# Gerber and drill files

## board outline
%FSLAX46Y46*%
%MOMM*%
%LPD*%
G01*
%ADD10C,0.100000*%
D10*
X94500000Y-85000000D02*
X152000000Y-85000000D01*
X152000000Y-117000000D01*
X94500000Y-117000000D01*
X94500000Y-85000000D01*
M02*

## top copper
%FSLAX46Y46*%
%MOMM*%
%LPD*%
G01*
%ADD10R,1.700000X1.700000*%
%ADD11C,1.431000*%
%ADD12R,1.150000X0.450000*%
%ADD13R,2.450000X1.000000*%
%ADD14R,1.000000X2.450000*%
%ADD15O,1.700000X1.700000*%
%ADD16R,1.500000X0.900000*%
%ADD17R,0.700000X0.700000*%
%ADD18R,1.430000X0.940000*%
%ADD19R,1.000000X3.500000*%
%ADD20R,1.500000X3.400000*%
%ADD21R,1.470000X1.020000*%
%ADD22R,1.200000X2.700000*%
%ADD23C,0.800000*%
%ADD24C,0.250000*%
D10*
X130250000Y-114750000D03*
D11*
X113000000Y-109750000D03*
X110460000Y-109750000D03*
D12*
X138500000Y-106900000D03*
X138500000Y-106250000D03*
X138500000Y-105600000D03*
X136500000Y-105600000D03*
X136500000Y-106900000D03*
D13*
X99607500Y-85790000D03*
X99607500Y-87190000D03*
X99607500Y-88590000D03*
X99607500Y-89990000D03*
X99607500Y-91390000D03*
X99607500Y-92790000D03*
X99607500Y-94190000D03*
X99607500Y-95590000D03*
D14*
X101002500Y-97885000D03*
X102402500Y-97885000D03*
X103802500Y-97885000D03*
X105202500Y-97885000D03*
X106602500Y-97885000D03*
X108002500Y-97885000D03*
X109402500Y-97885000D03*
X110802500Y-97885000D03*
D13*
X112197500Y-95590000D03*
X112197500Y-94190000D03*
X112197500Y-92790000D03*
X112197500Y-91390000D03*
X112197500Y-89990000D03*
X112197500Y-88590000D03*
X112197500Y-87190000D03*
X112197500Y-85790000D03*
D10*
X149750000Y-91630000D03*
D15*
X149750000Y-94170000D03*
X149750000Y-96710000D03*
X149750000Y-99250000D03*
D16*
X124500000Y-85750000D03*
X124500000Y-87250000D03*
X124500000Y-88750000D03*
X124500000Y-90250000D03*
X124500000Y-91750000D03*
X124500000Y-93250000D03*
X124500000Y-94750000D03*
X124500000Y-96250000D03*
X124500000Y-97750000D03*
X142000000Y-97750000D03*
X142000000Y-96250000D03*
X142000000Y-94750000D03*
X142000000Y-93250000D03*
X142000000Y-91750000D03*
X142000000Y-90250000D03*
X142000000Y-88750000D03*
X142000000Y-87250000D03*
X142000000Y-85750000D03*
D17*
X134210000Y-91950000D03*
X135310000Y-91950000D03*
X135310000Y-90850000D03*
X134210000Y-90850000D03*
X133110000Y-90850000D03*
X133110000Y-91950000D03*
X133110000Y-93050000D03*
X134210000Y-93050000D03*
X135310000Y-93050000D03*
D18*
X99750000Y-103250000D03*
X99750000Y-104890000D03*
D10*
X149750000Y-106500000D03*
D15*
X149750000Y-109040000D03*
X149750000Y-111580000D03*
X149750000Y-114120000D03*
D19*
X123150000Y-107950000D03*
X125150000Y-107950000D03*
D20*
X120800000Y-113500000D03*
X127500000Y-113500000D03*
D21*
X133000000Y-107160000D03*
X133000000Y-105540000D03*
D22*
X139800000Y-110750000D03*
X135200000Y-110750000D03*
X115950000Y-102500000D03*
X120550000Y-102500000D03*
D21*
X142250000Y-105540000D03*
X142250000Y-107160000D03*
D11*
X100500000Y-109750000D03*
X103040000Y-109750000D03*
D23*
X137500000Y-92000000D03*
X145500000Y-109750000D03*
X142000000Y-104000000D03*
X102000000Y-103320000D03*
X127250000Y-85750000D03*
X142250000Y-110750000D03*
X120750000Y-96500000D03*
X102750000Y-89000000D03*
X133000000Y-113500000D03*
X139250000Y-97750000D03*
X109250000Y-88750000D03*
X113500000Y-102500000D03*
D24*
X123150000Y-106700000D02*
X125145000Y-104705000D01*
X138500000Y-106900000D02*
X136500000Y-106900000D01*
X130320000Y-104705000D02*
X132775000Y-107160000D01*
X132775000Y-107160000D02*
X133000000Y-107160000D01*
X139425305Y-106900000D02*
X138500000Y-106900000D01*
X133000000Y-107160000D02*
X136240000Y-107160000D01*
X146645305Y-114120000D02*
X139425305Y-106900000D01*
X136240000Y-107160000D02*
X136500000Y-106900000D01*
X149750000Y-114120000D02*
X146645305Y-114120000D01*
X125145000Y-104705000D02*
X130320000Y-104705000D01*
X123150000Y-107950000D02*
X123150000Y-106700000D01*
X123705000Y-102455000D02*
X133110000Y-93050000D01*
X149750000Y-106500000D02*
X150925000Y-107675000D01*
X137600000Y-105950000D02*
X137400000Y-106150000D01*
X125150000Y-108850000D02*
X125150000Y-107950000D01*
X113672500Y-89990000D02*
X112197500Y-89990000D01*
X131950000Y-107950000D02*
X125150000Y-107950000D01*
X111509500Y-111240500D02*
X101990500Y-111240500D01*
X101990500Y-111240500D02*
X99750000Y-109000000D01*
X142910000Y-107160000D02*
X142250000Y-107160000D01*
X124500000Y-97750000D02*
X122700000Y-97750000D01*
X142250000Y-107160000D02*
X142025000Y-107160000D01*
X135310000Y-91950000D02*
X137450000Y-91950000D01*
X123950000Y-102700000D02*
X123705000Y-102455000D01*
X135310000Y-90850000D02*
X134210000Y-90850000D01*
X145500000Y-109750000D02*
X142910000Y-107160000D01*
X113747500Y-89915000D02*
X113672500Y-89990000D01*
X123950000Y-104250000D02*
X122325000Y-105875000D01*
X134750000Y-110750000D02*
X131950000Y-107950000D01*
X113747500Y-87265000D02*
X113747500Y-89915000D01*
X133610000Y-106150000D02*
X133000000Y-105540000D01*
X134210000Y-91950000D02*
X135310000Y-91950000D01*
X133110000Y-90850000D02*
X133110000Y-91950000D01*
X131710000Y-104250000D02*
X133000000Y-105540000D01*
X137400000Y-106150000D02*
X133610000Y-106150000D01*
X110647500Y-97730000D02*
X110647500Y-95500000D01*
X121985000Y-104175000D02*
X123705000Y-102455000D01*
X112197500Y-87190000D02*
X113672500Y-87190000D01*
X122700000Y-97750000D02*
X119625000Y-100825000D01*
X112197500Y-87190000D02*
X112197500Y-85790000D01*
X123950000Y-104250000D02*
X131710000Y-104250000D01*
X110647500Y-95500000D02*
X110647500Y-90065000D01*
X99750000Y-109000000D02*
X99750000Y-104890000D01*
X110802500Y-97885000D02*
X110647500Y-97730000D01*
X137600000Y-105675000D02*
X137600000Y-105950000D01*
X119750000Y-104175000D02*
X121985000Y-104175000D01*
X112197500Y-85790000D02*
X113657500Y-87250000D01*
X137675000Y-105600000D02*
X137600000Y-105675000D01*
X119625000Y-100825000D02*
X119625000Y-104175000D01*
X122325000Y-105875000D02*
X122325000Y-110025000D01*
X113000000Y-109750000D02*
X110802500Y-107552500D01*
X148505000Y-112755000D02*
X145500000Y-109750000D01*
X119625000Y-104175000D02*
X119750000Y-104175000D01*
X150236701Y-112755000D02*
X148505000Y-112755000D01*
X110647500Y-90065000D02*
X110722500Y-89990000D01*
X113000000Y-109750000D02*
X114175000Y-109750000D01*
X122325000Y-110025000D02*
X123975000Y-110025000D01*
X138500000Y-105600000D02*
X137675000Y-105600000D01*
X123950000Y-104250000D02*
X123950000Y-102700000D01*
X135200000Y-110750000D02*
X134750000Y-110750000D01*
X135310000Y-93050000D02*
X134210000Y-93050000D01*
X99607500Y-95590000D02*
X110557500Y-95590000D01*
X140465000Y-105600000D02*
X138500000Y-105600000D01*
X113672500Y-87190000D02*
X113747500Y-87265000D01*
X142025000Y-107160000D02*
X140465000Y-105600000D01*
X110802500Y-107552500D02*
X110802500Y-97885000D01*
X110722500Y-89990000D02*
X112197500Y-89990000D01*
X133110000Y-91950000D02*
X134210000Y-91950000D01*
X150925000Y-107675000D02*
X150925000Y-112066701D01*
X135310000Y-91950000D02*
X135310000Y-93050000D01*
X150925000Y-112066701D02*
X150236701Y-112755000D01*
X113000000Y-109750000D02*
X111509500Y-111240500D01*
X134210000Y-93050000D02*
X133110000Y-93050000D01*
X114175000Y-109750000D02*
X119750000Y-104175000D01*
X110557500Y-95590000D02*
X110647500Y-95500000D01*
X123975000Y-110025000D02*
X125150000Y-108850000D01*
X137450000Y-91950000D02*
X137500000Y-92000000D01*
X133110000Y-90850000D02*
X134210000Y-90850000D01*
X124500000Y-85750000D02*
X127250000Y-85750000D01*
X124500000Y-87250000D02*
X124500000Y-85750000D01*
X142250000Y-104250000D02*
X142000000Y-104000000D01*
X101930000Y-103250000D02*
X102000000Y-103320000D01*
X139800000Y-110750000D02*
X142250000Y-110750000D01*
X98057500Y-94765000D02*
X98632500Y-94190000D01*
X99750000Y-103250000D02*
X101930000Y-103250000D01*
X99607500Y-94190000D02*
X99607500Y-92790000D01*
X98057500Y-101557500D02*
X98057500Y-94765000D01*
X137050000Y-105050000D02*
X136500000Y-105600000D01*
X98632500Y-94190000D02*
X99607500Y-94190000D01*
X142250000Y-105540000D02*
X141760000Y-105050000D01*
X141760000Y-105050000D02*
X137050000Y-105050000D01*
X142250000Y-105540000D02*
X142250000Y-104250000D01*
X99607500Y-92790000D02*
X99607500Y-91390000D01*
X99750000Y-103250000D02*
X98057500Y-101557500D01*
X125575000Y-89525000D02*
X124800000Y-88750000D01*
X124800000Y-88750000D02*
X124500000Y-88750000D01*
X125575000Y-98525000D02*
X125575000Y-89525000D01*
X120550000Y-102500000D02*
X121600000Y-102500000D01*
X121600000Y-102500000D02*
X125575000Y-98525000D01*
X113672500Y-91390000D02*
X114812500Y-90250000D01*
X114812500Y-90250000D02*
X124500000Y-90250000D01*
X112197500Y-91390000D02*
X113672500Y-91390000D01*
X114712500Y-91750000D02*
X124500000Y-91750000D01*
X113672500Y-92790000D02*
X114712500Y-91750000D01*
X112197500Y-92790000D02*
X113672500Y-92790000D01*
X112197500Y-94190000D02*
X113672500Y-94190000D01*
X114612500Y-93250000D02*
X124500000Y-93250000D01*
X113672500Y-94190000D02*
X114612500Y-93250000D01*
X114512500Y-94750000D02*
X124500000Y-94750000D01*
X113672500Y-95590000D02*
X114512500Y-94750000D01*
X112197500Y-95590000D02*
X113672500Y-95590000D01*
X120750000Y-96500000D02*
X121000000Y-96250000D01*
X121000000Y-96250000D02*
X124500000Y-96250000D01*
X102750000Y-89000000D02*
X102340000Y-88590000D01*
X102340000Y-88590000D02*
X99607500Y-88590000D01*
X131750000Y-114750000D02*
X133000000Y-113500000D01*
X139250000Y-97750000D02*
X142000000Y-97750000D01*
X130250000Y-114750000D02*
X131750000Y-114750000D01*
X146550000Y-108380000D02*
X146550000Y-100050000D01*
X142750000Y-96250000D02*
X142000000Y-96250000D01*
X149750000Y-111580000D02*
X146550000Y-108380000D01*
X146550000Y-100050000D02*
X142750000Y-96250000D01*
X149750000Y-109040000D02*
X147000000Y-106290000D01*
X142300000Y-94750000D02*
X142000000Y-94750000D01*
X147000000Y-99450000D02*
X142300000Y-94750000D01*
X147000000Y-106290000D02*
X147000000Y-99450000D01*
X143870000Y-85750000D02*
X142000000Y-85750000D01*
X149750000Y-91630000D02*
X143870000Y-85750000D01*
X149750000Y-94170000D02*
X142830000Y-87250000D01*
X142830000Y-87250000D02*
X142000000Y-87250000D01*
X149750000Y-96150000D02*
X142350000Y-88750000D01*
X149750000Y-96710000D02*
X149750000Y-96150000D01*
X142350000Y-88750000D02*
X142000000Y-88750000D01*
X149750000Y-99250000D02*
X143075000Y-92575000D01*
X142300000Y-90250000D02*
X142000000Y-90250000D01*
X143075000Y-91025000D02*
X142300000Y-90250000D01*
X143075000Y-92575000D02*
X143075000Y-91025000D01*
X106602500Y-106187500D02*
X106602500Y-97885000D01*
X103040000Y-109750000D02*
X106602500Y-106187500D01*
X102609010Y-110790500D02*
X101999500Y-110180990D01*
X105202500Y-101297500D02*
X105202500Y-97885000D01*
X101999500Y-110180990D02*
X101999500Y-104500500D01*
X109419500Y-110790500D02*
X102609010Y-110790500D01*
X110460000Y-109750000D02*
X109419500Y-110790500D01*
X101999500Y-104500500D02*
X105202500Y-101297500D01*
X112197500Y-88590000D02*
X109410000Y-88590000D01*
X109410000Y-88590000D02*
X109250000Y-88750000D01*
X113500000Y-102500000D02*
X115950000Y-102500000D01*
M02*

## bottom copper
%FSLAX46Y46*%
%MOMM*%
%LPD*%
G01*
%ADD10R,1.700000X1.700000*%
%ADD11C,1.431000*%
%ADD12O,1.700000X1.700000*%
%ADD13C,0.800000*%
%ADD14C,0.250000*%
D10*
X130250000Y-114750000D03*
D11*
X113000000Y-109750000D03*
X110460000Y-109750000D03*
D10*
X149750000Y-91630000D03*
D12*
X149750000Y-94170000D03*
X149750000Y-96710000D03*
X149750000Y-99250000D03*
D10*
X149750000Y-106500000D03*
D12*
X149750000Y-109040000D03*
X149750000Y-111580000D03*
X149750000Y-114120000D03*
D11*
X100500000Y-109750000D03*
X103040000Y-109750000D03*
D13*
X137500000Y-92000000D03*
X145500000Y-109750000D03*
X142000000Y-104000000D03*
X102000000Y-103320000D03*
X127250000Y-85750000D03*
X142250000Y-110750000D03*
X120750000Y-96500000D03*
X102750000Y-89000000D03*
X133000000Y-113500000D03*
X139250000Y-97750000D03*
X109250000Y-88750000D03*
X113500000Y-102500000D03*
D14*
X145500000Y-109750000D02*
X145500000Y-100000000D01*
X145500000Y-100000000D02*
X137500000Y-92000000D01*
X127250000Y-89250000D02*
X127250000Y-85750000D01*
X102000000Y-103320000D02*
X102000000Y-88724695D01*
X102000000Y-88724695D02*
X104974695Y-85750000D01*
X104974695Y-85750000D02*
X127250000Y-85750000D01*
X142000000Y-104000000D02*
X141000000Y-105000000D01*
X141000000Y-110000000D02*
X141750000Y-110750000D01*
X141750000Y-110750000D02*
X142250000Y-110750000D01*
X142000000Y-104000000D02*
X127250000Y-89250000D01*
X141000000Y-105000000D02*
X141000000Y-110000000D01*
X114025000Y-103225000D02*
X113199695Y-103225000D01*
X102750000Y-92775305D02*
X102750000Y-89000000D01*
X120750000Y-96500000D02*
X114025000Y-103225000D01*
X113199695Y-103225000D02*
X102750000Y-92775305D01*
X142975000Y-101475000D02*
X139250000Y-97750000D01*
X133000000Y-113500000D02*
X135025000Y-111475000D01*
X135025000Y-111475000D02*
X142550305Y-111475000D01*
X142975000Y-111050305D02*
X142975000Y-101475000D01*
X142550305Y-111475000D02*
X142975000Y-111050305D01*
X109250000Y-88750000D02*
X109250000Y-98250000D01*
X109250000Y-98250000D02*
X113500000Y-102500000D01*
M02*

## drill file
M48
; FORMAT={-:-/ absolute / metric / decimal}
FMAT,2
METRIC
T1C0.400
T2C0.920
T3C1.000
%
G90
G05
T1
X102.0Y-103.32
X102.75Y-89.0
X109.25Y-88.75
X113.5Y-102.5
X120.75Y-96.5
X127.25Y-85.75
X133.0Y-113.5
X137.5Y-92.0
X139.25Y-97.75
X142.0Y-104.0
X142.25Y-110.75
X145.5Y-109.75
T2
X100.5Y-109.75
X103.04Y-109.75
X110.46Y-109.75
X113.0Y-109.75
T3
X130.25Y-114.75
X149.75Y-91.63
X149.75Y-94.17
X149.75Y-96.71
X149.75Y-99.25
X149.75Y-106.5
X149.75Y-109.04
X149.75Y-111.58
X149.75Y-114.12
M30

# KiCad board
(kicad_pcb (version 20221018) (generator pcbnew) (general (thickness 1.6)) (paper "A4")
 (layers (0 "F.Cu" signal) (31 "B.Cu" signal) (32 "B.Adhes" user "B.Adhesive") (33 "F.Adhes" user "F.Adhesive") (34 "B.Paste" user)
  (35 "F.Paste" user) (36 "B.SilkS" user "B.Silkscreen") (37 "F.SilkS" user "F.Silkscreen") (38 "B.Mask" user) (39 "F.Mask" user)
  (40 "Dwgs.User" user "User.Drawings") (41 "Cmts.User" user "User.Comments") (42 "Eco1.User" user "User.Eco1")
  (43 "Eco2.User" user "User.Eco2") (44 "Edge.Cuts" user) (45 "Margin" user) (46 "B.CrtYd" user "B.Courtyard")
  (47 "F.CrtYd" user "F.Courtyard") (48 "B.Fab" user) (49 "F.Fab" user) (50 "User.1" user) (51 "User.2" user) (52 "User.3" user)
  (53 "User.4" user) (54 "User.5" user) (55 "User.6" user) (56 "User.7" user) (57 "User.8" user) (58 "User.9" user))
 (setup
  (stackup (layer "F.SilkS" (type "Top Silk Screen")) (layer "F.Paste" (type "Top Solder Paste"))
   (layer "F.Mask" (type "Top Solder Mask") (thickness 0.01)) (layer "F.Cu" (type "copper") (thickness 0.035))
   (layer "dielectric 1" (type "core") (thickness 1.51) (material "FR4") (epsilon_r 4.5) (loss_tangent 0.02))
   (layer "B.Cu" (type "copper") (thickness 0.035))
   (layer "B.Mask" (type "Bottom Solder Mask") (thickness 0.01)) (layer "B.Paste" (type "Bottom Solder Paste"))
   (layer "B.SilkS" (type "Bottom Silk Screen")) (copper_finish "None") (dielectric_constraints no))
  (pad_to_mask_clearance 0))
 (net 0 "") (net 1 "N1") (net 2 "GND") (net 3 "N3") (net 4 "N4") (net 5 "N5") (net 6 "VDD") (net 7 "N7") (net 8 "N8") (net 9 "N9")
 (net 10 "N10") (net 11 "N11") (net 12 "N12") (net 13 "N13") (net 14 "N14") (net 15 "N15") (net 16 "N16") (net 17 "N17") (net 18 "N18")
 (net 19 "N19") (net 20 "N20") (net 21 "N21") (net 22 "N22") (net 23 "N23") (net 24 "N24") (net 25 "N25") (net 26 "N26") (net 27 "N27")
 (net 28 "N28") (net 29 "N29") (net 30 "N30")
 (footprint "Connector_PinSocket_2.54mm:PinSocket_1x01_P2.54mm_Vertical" (layer "F.Cu") (at 130.25 114.75)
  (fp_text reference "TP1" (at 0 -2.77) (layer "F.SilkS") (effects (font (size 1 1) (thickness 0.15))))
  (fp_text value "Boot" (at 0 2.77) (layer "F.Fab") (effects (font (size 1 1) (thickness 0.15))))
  (pad "1" thru_hole rect (at 0 0) (size 1.7 1.7) (drill 1) (layers "*.Cu" "*.Mask") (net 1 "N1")))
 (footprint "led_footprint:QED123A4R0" (layer "F.Cu") (at 113 109.75)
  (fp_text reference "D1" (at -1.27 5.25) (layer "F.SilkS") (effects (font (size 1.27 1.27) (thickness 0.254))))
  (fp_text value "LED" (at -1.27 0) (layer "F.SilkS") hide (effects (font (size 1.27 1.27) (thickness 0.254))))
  (pad "1" thru_hole circle (at 0 0) (size 1.431 1.431) (drill 0.92) (layers "*.Cu" "*.Mask") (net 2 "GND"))
  (pad "2" thru_hole circle (at -2.54 0) (size 1.431 1.431) (drill 0.92) (layers "*.Cu" "*.Mask") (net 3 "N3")))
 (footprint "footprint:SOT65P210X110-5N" (layer "F.Cu") (at 137.5 106.25 180)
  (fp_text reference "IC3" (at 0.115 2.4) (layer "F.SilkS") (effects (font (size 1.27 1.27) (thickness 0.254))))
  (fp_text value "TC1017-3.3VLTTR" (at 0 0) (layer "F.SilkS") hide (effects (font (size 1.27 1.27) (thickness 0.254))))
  (pad "1" smd rect (at -1 -0.65 270) (size 0.45 1.15) (layers "F.Cu" "F.Paste" "F.Mask") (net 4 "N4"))
  (pad "2" smd rect (at -1 0 270) (size 0.45 1.15) (layers "F.Cu" "F.Paste" "F.Mask") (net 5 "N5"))
  (pad "3" smd rect (at -1 0.65 270) (size 0.45 1.15) (layers "F.Cu" "F.Paste" "F.Mask") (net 2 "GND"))
  (pad "4" smd rect (at 1 0.65 270) (size 0.45 1.15) (layers "F.Cu" "F.Paste" "F.Mask") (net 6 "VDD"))
  (pad "5" smd rect (at 1 -0.65 270) (size 0.45 1.15) (layers "F.Cu" "F.Paste" "F.Mask") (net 4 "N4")))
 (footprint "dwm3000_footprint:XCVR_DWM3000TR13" (layer "F.Cu") (at 105.9025 86.74)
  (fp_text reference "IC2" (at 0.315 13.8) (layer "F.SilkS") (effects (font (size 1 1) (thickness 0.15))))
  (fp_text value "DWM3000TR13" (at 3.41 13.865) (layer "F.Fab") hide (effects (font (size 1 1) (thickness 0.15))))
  (pad "1" smd rect (at -6.295 -0.95) (size 2.45 1) (layers "F.Cu" "F.Paste" "F.Mask") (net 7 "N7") (solder_mask_margin 0.102))
  (pad "2" smd rect (at -6.295 0.45) (size 2.45 1) (layers "F.Cu" "F.Paste" "F.Mask") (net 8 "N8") (solder_mask_margin 0.102))
  (pad "3" smd rect (at -6.295 1.85) (size 2.45 1) (layers "F.Cu" "F.Paste" "F.Mask") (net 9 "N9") (solder_mask_margin 0.102))
  (pad "4" smd rect (at -6.295 3.25) (size 2.45 1) (layers "F.Cu" "F.Paste" "F.Mask") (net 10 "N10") (solder_mask_margin 0.102))
  (pad "5" smd rect (at -6.295 4.65) (size 2.45 1) (layers "F.Cu" "F.Paste" "F.Mask") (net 6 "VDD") (solder_mask_margin 0.102))
  (pad "6" smd rect (at -6.295 6.05) (size 2.45 1) (layers "F.Cu" "F.Paste" "F.Mask") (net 6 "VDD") (solder_mask_margin 0.102))
  (pad "7" smd rect (at -6.295 7.45) (size 2.45 1) (layers "F.Cu" "F.Paste" "F.Mask") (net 6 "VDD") (solder_mask_margin 0.102))
  (pad "8" smd rect (at -6.295 8.85) (size 2.45 1) (layers "F.Cu" "F.Paste" "F.Mask") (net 2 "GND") (solder_mask_margin 0.102))
  (pad "9" smd rect (at -4.9 11.145) (size 1 2.45) (layers "F.Cu" "F.Paste" "F.Mask") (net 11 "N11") (solder_mask_margin 0.102))
  (pad "10" smd rect (at -3.5 11.145) (size 1 2.45) (layers "F.Cu" "F.Paste" "F.Mask") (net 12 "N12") (solder_mask_margin 0.102))
  (pad "11" smd rect (at -2.1 11.145) (size 1 2.45) (layers "F.Cu" "F.Paste" "F.Mask") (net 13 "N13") (solder_mask_margin 0.102))
  (pad "12" smd rect (at -0.7 11.145) (size 1 2.45) (layers "F.Cu" "F.Paste" "F.Mask") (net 3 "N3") (solder_mask_margin 0.102))
  (pad "13" smd rect (at 0.7 11.145) (size 1 2.45) (layers "F.Cu" "F.Paste" "F.Mask") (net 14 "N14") (solder_mask_margin 0.102))
  (pad "14" smd rect (at 2.1 11.145) (size 1 2.45) (layers "F.Cu" "F.Paste" "F.Mask") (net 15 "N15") (solder_mask_margin 0.102))
  (pad "15" smd rect (at 3.5 11.145) (size 1 2.45) (layers "F.Cu" "F.Paste" "F.Mask") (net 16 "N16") (solder_mask_margin 0.102))
  (pad "16" smd rect (at 4.9 11.145) (size 1 2.45) (layers "F.Cu" "F.Paste" "F.Mask") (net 2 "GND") (solder_mask_margin 0.102))
  (pad "17" smd rect (at 6.295 8.85) (size 2.45 1) (layers "F.Cu" "F.Paste" "F.Mask") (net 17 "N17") (solder_mask_margin 0.102))
  (pad "18" smd rect (at 6.295 7.45) (size 2.45 1) (layers "F.Cu" "F.Paste" "F.Mask") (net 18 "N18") (solder_mask_margin 0.102))
  (pad "19" smd rect (at 6.295 6.05) (size 2.45 1) (layers "F.Cu" "F.Paste" "F.Mask") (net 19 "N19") (solder_mask_margin 0.102))
  (pad "20" smd rect (at 6.295 4.65) (size 2.45 1) (layers "F.Cu" "F.Paste" "F.Mask") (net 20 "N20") (solder_mask_margin 0.102))
  (pad "21" smd rect (at 6.295 3.25) (size 2.45 1) (layers "F.Cu" "F.Paste" "F.Mask") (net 2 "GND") (solder_mask_margin 0.102))
  (pad "22" smd rect (at 6.295 1.85) (size 2.45 1) (layers "F.Cu" "F.Paste" "F.Mask") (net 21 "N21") (solder_mask_margin 0.102))
  (pad "23" smd rect (at 6.295 0.45) (size 2.45 1) (layers "F.Cu" "F.Paste" "F.Mask") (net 2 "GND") (solder_mask_margin 0.102))
  (pad "24" smd rect (at 6.295 -0.95) (size 2.45 1) (layers "F.Cu" "F.Paste" "F.Mask") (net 2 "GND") (solder_mask_margin 0.102))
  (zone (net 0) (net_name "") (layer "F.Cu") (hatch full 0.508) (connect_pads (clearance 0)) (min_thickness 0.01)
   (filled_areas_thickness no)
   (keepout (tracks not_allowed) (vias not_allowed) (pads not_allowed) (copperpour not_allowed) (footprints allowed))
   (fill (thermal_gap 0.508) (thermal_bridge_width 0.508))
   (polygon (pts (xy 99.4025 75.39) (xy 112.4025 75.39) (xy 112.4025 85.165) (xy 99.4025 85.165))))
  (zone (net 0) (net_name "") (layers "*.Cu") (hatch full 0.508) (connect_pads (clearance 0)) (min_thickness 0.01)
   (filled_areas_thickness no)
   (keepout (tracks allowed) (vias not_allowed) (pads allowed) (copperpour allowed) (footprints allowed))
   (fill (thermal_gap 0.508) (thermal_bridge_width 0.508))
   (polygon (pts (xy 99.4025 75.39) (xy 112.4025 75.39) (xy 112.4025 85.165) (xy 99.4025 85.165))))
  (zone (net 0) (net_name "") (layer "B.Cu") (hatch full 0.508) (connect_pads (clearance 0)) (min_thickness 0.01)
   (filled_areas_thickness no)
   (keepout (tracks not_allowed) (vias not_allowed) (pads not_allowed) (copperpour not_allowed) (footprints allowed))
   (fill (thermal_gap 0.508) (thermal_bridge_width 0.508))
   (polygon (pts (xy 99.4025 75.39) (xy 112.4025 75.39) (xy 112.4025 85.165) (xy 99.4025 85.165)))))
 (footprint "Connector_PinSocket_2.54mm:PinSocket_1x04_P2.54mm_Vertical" (layer "F.Cu") (at 149.75 91.63)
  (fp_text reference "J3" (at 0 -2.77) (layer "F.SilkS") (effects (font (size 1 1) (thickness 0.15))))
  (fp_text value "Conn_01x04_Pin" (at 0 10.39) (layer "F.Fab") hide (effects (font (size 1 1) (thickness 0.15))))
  (pad "1" thru_hole rect (at 0 0) (size 1.7 1.7) (drill 1) (layers "*.Cu" "*.Mask") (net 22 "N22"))
  (pad "2" thru_hole oval (at 0 2.54) (size 1.7 1.7) (drill 1) (layers "*.Cu" "*.Mask") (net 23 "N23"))
  (pad "3" thru_hole oval (at 0 5.08) (size 1.7 1.7) (drill 1) (layers "*.Cu" "*.Mask") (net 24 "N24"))
  (pad "4" thru_hole oval (at 0 7.62) (size 1.7 1.7) (drill 1) (layers "*.Cu" "*.Mask") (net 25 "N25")))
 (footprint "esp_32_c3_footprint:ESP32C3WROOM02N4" (layer "F.Cu") (at 134.21 91.95)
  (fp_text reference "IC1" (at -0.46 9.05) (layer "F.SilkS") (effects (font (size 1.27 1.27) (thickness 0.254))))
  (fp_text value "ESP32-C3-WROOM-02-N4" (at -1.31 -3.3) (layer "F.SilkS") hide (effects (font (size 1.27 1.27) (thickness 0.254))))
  (pad "1" smd rect (at -9.71 -6.2 90) (size 0.9 1.5) (layers "F.Cu" "F.Paste" "F.Mask") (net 6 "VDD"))
  (pad "2" smd rect (at -9.71 -4.7 90) (size 0.9 1.5) (layers "F.Cu" "F.Paste" "F.Mask") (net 6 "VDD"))
  (pad "3" smd rect (at -9.71 -3.2 90) (size 0.9 1.5) (layers "F.Cu" "F.Paste" "F.Mask") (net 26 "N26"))
  (pad "4" smd rect (at -9.71 -1.7 90) (size 0.9 1.5) (layers "F.Cu" "F.Paste" "F.Mask") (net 20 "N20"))
  (pad "5" smd rect (at -9.71 -0.2 90) (size 0.9 1.5) (layers "F.Cu" "F.Paste" "F.Mask") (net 19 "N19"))
  (pad "6" smd rect (at -9.71 1.3 90) (size 0.9 1.5) (layers "F.Cu" "F.Paste" "F.Mask") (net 18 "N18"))
  (pad "7" smd rect (at -9.71 2.8 90) (size 0.9 1.5) (layers "F.Cu" "F.Paste" "F.Mask") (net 17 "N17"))
  (pad "8" smd rect (at -9.71 4.3 90) (size 0.9 1.5) (layers "F.Cu" "F.Paste" "F.Mask") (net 9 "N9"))
  (pad "9" smd rect (at -9.71 5.8 90) (size 0.9 1.5) (layers "F.Cu" "F.Paste" "F.Mask") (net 2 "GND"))
  (pad "10" smd rect (at 7.79 5.8 90) (size 0.9 1.5) (layers "F.Cu" "F.Paste" "F.Mask") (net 1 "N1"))
  (pad "11" smd rect (at 7.79 4.3 90) (size 0.9 1.5) (layers "F.Cu" "F.Paste" "F.Mask") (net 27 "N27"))
  (pad "12" smd rect (at 7.79 2.8 90) (size 0.9 1.5) (layers "F.Cu" "F.Paste" "F.Mask") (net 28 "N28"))
  (pad "13" smd rect (at 7.79 1.3 90) (size 0.9 1.5) (layers "F.Cu" "F.Paste" "F.Mask") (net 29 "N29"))
  (pad "14" smd rect (at 7.79 -0.2 90) (size 0.9 1.5) (layers "F.Cu" "F.Paste" "F.Mask") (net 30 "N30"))
  (pad "15" smd rect (at 7.79 -1.7 90) (size 0.9 1.5) (layers "F.Cu" "F.Paste" "F.Mask") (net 25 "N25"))
  (pad "16" smd rect (at 7.79 -3.2 90) (size 0.9 1.5) (layers "F.Cu" "F.Paste" "F.Mask") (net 24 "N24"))
  (pad "17" smd rect (at 7.79 -4.7 90) (size 0.9 1.5) (layers "F.Cu" "F.Paste" "F.Mask") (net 23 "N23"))
  (pad "18" smd rect (at 7.79 -6.2 90) (size 0.9 1.5) (layers "F.Cu" "F.Paste" "F.Mask") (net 22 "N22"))
  (pad "19" smd rect (at 0 0 90) (size 0.7 0.7) (layers "F.Cu" "F.Paste" "F.Mask") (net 2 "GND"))
  (pad "20" smd rect (at 1.1 0 90) (size 0.7 0.7) (layers "F.Cu" "F.Paste" "F.Mask") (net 2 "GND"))
  (pad "21" smd rect (at 1.1 -1.1 90) (size 0.7 0.7) (layers "F.Cu" "F.Paste" "F.Mask") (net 2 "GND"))
  (pad "22" smd rect (at 0 -1.1 90) (size 0.7 0.7) (layers "F.Cu" "F.Paste" "F.Mask") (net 2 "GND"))
  (pad "23" smd rect (at -1.1 -1.1 90) (size 0.7 0.7) (layers "F.Cu" "F.Paste" "F.Mask") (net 2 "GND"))
  (pad "24" smd rect (at -1.1 0 90) (size 0.7 0.7) (layers "F.Cu" "F.Paste" "F.Mask") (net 2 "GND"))
  (pad "25" smd rect (at -1.1 1.1 90) (size 0.7 0.7) (layers "F.Cu" "F.Paste" "F.Mask") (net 2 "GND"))
  (pad "26" smd rect (at 0 1.1 90) (size 0.7 0.7) (layers "F.Cu" "F.Paste" "F.Mask") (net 2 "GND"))
  (pad "27" smd rect (at 1.1 1.1 90) (size 0.7 0.7) (layers "F.Cu" "F.Paste" "F.Mask") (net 2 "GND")))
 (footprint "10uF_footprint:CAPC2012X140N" (layer "F.Cu") (at 99.75 104.07 -90)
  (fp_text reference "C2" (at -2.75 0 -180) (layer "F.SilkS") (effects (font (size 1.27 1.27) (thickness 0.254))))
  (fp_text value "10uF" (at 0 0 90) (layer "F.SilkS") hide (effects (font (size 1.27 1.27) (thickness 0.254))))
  (pad "1" smd rect (at -0.82 0 270) (size 0.94 1.43) (layers "F.Cu" "F.Paste" "F.Mask") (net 6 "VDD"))
  (pad "2" smd rect (at 0.82 0 270) (size 0.94 1.43) (layers "F.Cu" "F.Paste" "F.Mask") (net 2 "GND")))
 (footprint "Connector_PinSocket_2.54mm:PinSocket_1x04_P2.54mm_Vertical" (layer "F.Cu") (at 149.75 106.5)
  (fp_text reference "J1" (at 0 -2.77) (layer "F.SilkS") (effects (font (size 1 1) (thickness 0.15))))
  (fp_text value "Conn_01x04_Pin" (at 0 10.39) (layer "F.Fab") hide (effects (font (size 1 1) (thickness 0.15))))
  (pad "1" thru_hole rect (at 0 0) (size 1.7 1.7) (drill 1) (layers "*.Cu" "*.Mask") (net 2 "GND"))
  (pad "2" thru_hole oval (at 0 2.54) (size 1.7 1.7) (drill 1) (layers "*.Cu" "*.Mask") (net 28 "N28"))
  (pad "3" thru_hole oval (at 0 5.08) (size 1.7 1.7) (drill 1) (layers "*.Cu" "*.Mask") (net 27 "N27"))
  (pad "4" thru_hole oval (at 0 7.62) (size 1.7 1.7) (drill 1) (layers "*.Cu" "*.Mask") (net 4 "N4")))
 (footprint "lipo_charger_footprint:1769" (layer "F.Cu") (at 124.15 107.95)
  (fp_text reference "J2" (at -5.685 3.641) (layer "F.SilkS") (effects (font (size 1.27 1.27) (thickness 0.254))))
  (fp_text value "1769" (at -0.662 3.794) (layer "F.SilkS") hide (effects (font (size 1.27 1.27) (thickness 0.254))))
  (pad "1" smd rect (at -1 0) (size 1 3.5) (layers "F.Cu" "F.Paste" "F.Mask") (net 4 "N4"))
  (pad "2" smd rect (at 1 0) (size 1 3.5) (layers "F.Cu" "F.Paste" "F.Mask") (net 2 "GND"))
  (pad "3" smd rect (at -3.35 5.55) (size 1.5 3.4) (layers "F.Cu" "F.Paste" "F.Mask"))
  (pad "4" smd rect (at 3.35 5.55) (size 1.5 3.4) (layers "F.Cu" "F.Paste" "F.Mask")))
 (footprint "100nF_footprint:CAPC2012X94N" (layer "F.Cu") (at 133 106.35 90)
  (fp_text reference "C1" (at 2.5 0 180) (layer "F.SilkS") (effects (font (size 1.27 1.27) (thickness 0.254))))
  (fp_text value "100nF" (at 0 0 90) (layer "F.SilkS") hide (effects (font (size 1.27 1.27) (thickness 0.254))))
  (pad "1" smd rect (at -0.81 0 90) (size 1.02 1.47) (layers "F.Cu" "F.Paste" "F.Mask") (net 4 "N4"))
  (pad "2" smd rect (at 0.81 0 90) (size 1.02 1.47) (layers "F.Cu" "F.Paste" "F.Mask") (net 2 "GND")))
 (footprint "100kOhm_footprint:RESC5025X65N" (layer "F.Cu") (at 137.5 110.75 180)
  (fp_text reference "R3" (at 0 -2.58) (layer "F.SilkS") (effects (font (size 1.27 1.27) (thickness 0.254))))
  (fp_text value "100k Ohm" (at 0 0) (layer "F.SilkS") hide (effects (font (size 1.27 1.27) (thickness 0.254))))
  (pad "1" smd rect (at -2.3 0 180) (size 1.2 2.7) (layers "F.Cu" "F.Paste" "F.Mask") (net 6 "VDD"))
  (pad "2" smd rect (at 2.3 0 180) (size 1.2 2.7) (layers "F.Cu" "F.Paste" "F.Mask") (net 2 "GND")))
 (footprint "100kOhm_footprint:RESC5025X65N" (layer "F.Cu") (at 118.25 102.5)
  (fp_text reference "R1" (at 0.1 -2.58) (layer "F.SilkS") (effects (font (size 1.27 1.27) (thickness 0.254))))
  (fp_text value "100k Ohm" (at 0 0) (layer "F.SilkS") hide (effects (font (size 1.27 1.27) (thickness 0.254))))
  (pad "1" smd rect (at -2.3 0) (size 1.2 2.7) (layers "F.Cu" "F.Paste" "F.Mask") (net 21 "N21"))
  (pad "2" smd rect (at 2.3 0) (size 1.2 2.7) (layers "F.Cu" "F.Paste" "F.Mask") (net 26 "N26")))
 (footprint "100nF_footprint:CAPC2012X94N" (layer "F.Cu") (at 142.25 106.35 -90)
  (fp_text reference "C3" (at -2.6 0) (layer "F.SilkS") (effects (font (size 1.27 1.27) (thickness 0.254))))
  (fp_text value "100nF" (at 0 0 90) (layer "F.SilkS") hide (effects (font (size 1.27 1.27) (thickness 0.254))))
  (pad "1" smd rect (at -0.81 0 270) (size 1.02 1.47) (layers "F.Cu" "F.Paste" "F.Mask") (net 6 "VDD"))
  (pad "2" smd rect (at 0.81 0 270) (size 1.02 1.47) (layers "F.Cu" "F.Paste" "F.Mask") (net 2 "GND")))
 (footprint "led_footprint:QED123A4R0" (layer "B.Cu") (at 100.5 109.75 180)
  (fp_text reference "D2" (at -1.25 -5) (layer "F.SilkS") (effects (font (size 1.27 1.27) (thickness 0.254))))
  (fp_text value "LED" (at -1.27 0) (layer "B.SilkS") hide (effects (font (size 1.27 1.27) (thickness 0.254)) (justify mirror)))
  (pad "1" thru_hole circle (at 0 0 180) (size 1.431 1.431) (drill 0.92) (layers "*.Cu" "*.Mask") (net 2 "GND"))
  (pad "2" thru_hole circle (at -2.54 0 180) (size 1.431 1.431) (drill 0.92) (layers "*.Cu" "*.Mask") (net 14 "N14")))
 (gr_rect (start 94.5 85) (end 152 117) (stroke (width 0.1) (type default)) (fill none) (layer "Edge.Cuts"))
 (segment (start 123.15 106.7) (end 125.145 104.705) (width 0.25) (layer "F.Cu") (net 4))
 (segment (start 138.5 106.9) (end 136.5 106.9) (width 0.25) (layer "F.Cu") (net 4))
 (segment (start 130.32 104.705) (end 132.775 107.16) (width 0.25) (layer "F.Cu") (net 4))
 (segment (start 132.775 107.16) (end 133 107.16) (width 0.25) (layer "F.Cu") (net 4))
 (segment (start 139.425305 106.9) (end 138.5 106.9) (width 0.25) (layer "F.Cu") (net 4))
 (segment (start 133 107.16) (end 136.24 107.16) (width 0.25) (layer "F.Cu") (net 4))
 (segment (start 146.645305 114.12) (end 139.425305 106.9) (width 0.25) (layer "F.Cu") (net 4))
 (segment (start 136.24 107.16) (end 136.5 106.9) (width 0.25) (layer "F.Cu") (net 4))
 (segment (start 149.75 114.12) (end 146.645305 114.12) (width 0.25) (layer "F.Cu") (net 4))
 (segment (start 125.145 104.705) (end 130.32 104.705) (width 0.25) (layer "F.Cu") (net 4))
 (segment (start 123.15 107.95) (end 123.15 106.7) (width 0.25) (layer "F.Cu") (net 4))
 (segment (start 123.705 102.455) (end 133.11 93.05) (width 0.25) (layer "F.Cu") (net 2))
 (segment (start 149.75 106.5) (end 150.925 107.675) (width 0.25) (layer "F.Cu") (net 2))
 (segment (start 137.6 105.95) (end 137.4 106.15) (width 0.25) (layer "F.Cu") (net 2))
 (segment (start 125.15 108.85) (end 125.15 107.95) (width 0.25) (layer "F.Cu") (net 2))
 (segment (start 113.6725 89.99) (end 112.1975 89.99) (width 0.25) (layer "F.Cu") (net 2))
 (segment (start 131.95 107.95) (end 125.15 107.95) (width 0.25) (layer "F.Cu") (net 2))
 (segment (start 111.5095 111.2405) (end 101.9905 111.2405) (width 0.25) (layer "F.Cu") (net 2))
 (segment (start 101.9905 111.2405) (end 99.75 109) (width 0.25) (layer "F.Cu") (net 2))
 (segment (start 142.91 107.16) (end 142.25 107.16) (width 0.25) (layer "F.Cu") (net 2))
 (segment (start 124.5 97.75) (end 122.7 97.75) (width 0.25) (layer "F.Cu") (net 2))
 (segment (start 142.25 107.16) (end 142.025 107.16) (width 0.25) (layer "F.Cu") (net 2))
 (segment (start 135.31 91.95) (end 137.45 91.95) (width 0.25) (layer "F.Cu") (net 2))
 (segment (start 123.95 102.7) (end 123.705 102.455) (width 0.25) (layer "F.Cu") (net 2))
 (segment (start 135.31 90.85) (end 134.21 90.85) (width 0.25) (layer "F.Cu") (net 2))
 (segment (start 145.5 109.75) (end 142.91 107.16) (width 0.25) (layer "F.Cu") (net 2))
 (segment (start 113.7475 89.915) (end 113.6725 89.99) (width 0.25) (layer "F.Cu") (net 2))
 (segment (start 123.95 104.25) (end 122.325 105.875) (width 0.25) (layer "F.Cu") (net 2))
 (segment (start 134.75 110.75) (end 131.95 107.95) (width 0.25) (layer "F.Cu") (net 2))
 (segment (start 113.7475 87.265) (end 113.7475 89.915) (width 0.25) (layer "F.Cu") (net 2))
 (segment (start 133.61 106.15) (end 133 105.54) (width 0.25) (layer "F.Cu") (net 2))
 (segment (start 134.21 91.95) (end 135.31 91.95) (width 0.25) (layer "F.Cu") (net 2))
 (segment (start 133.11 90.85) (end 133.11 91.95) (width 0.25) (layer "F.Cu") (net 2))
 (segment (start 131.71 104.25) (end 133 105.54) (width 0.25) (layer "F.Cu") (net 2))
 (segment (start 137.4 106.15) (end 133.61 106.15) (width 0.25) (layer "F.Cu") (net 2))
 (segment (start 110.6475 97.73) (end 110.6475 95.5) (width 0.25) (layer "F.Cu") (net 2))
 (segment (start 121.985 104.175) (end 123.705 102.455) (width 0.25) (layer "F.Cu") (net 2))
 (segment (start 112.1975 87.19) (end 113.6725 87.19) (width 0.25) (layer "F.Cu") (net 2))
 (segment (start 122.7 97.75) (end 119.625 100.825) (width 0.25) (layer "F.Cu") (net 2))
 (segment (start 112.1975 87.19) (end 112.1975 85.79) (width 0.25) (layer "F.Cu") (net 2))
 (segment (start 123.95 104.25) (end 131.71 104.25) (width 0.25) (layer "F.Cu") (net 2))
 (segment (start 110.6475 95.5) (end 110.6475 90.065) (width 0.25) (layer "F.Cu") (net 2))
 (segment (start 99.75 109) (end 99.75 104.89) (width 0.25) (layer "F.Cu") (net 2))
 (segment (start 110.8025 97.885) (end 110.6475 97.73) (width 0.25) (layer "F.Cu") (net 2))
 (segment (start 137.6 105.675) (end 137.6 105.95) (width 0.25) (layer "F.Cu") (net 2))
 (segment (start 119.75 104.175) (end 121.985 104.175) (width 0.25) (layer "F.Cu") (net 2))
 (segment (start 112.1975 85.79) (end 113.6575 87.25) (width 0.25) (layer "F.Cu") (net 2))
 (segment (start 137.675 105.6) (end 137.6 105.675) (width 0.25) (layer "F.Cu") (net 2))
 (segment (start 119.625 100.825) (end 119.625 104.175) (width 0.25) (layer "F.Cu") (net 2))
 (segment (start 122.325 105.875) (end 122.325 110.025) (width 0.25) (layer "F.Cu") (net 2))
 (segment (start 113 109.75) (end 110.8025 107.5525) (width 0.25) (layer "F.Cu") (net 2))
 (segment (start 148.505 112.755) (end 145.5 109.75) (width 0.25) (layer "F.Cu") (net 2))
 (segment (start 119.625 104.175) (end 119.75 104.175) (width 0.25) (layer "F.Cu") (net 2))
 (segment (start 150.236701 112.755) (end 148.505 112.755) (width 0.25) (layer "F.Cu") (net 2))
 (segment (start 110.6475 90.065) (end 110.7225 89.99) (width 0.25) (layer "F.Cu") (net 2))
 (segment (start 113 109.75) (end 114.175 109.75) (width 0.25) (layer "F.Cu") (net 2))
 (segment (start 122.325 110.025) (end 123.975 110.025) (width 0.25) (layer "F.Cu") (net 2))
 (segment (start 138.5 105.6) (end 137.675 105.6) (width 0.25) (layer "F.Cu") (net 2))
 (segment (start 123.95 104.25) (end 123.95 102.7) (width 0.25) (layer "F.Cu") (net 2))
 (segment (start 135.2 110.75) (end 134.75 110.75) (width 0.25) (layer "F.Cu") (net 2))
 (segment (start 135.31 93.05) (end 134.21 93.05) (width 0.25) (layer "F.Cu") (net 2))
 (segment (start 99.6075 95.59) (end 110.5575 95.59) (width 0.25) (layer "F.Cu") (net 2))
 (segment (start 140.465 105.6) (end 138.5 105.6) (width 0.25) (layer "F.Cu") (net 2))
 (segment (start 113.6725 87.19) (end 113.7475 87.265) (width 0.25) (layer "F.Cu") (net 2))
 (segment (start 142.025 107.16) (end 140.465 105.6) (width 0.25) (layer "F.Cu") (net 2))
 (segment (start 110.8025 107.5525) (end 110.8025 97.885) (width 0.25) (layer "F.Cu") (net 2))
 (segment (start 110.7225 89.99) (end 112.1975 89.99) (width 0.25) (layer "F.Cu") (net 2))
 (segment (start 133.11 91.95) (end 134.21 91.95) (width 0.25) (layer "F.Cu") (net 2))
 (segment (start 150.925 107.675) (end 150.925 112.066701) (width 0.25) (layer "F.Cu") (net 2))
 (segment (start 135.31 91.95) (end 135.31 93.05) (width 0.25) (layer "F.Cu") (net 2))
 (segment (start 150.925 112.066701) (end 150.236701 112.755) (width 0.25) (layer "F.Cu") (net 2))
 (segment (start 113 109.75) (end 111.5095 111.2405) (width 0.25) (layer "F.Cu") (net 2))
 (segment (start 134.21 93.05) (end 133.11 93.05) (width 0.25) (layer "F.Cu") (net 2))
 (segment (start 114.175 109.75) (end 119.75 104.175) (width 0.25) (layer "F.Cu") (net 2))
 (segment (start 110.5575 95.59) (end 110.6475 95.5) (width 0.25) (layer "F.Cu") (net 2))
 (segment (start 123.975 110.025) (end 125.15 108.85) (width 0.25) (layer "F.Cu") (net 2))
 (segment (start 137.45 91.95) (end 137.5 92) (width 0.25) (layer "F.Cu") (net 2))
 (segment (start 133.11 90.85) (end 134.21 90.85) (width 0.25) (layer "F.Cu") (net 2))
 (via blind (at 137.5 92) (size 0.8) (drill 0.4) (layers "F.Cu" "B.Cu") (free) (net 2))
 (via blind (at 145.5 109.75) (size 0.8) (drill 0.4) (layers "F.Cu" "B.Cu") (free) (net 2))
 (segment (start 145.5 109.75) (end 145.5 100) (width 0.25) (layer "B.Cu") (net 2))
 (segment (start 145.5 100) (end 137.5 92) (width 0.25) (layer "B.Cu") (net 2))
 (segment (start 124.5 85.75) (end 127.25 85.75) (width 0.25) (layer "F.Cu") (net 6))
 (segment (start 124.5 87.25) (end 124.5 85.75) (width 0.25) (layer "F.Cu") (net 6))
 (segment (start 142.25 104.25) (end 142 104) (width 0.25) (layer "F.Cu") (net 6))
 (segment (start 101.93 103.25) (end 102 103.32) (width 0.25) (layer "F.Cu") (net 6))
 (segment (start 139.8 110.75) (end 142.25 110.75) (width 0.25) (layer "F.Cu") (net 6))
 (segment (start 98.0575 94.765) (end 98.6325 94.19) (width 0.25) (layer "F.Cu") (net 6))
 (segment (start 99.75 103.25) (end 101.93 103.25) (width 0.25) (layer "F.Cu") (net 6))
 (segment (start 99.6075 94.19) (end 99.6075 92.79) (width 0.25) (layer "F.Cu") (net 6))
 (segment (start 98.0575 101.5575) (end 98.0575 94.765) (width 0.25) (layer "F.Cu") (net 6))
 (segment (start 137.05 105.05) (end 136.5 105.6) (width 0.25) (layer "F.Cu") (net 6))
 (segment (start 98.6325 94.19) (end 99.6075 94.19) (width 0.25) (layer "F.Cu") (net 6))
 (segment (start 142.25 105.54) (end 141.76 105.05) (width 0.25) (layer "F.Cu") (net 6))
 (segment (start 141.76 105.05) (end 137.05 105.05) (width 0.25) (layer "F.Cu") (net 6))
 (segment (start 142.25 105.54) (end 142.25 104.25) (width 0.25) (layer "F.Cu") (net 6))
 (segment (start 99.6075 92.79) (end 99.6075 91.39) (width 0.25) (layer "F.Cu") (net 6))
 (segment (start 99.75 103.25) (end 98.0575 101.5575) (width 0.25) (layer "F.Cu") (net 6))
 (via blind (at 142 104) (size 0.8) (drill 0.4) (layers "F.Cu" "B.Cu") (free) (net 6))
 (via blind (at 102 103.32) (size 0.8) (drill 0.4) (layers "F.Cu" "B.Cu") (free) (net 6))
 (via blind (at 127.25 85.75) (size 0.8) (drill 0.4) (layers "F.Cu" "B.Cu") (free) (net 6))
 (via blind (at 142.25 110.75) (size 0.8) (drill 0.4) (layers "F.Cu" "B.Cu") (free) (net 6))
 (segment (start 127.25 89.25) (end 127.25 85.75) (width 0.25) (layer "B.Cu") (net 6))
 (segment (start 102 103.32) (end 102 88.724695) (width 0.25) (layer "B.Cu") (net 6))
 (segment (start 102 88.724695) (end 104.974695 85.75) (width 0.25) (layer "B.Cu") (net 6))
 (segment (start 104.974695 85.75) (end 127.25 85.75) (width 0.25) (layer "B.Cu") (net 6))
 (segment (start 142 104) (end 141 105) (width 0.25) (layer "B.Cu") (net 6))
 (segment (start 141 110) (end 141.75 110.75) (width 0.25) (layer "B.Cu") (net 6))
 (segment (start 141.75 110.75) (end 142.25 110.75) (width 0.25) (layer "B.Cu") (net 6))
 (segment (start 142 104) (end 127.25 89.25) (width 0.25) (layer "B.Cu") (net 6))
 (segment (start 141 105) (end 141 110) (width 0.25) (layer "B.Cu") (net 6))
 (segment (start 125.575 89.525) (end 124.8 88.75) (width 0.25) (layer "F.Cu") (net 26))
 (segment (start 124.8 88.75) (end 124.5 88.75) (width 0.25) (layer "F.Cu") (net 26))
 (segment (start 125.575 98.525) (end 125.575 89.525) (width 0.25) (layer "F.Cu") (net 26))
 (segment (start 120.55 102.5) (end 121.6 102.5) (width 0.25) (layer "F.Cu") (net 26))
 (segment (start 121.6 102.5) (end 125.575 98.525) (width 0.25) (layer "F.Cu") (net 26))
 (segment (start 113.6725 91.39) (end 114.8125 90.25) (width 0.25) (layer "F.Cu") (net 20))
 (segment (start 114.8125 90.25) (end 124.5 90.25) (width 0.25) (layer "F.Cu") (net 20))
 (segment (start 112.1975 91.39) (end 113.6725 91.39) (width 0.25) (layer "F.Cu") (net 20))
 (segment (start 114.7125 91.75) (end 124.5 91.75) (width 0.25) (layer "F.Cu") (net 19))
 (segment (start 113.6725 92.79) (end 114.7125 91.75) (width 0.25) (layer "F.Cu") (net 19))
 (segment (start 112.1975 92.79) (end 113.6725 92.79) (width 0.25) (layer "F.Cu") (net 19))
 (segment (start 112.1975 94.19) (end 113.6725 94.19) (width 0.25) (layer "F.Cu") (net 18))
 (segment (start 114.6125 93.25) (end 124.5 93.25) (width 0.25) (layer "F.Cu") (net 18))
 (segment (start 113.6725 94.19) (end 114.6125 93.25) (width 0.25) (layer "F.Cu") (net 18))
 (segment (start 114.5125 94.75) (end 124.5 94.75) (width 0.25) (layer "F.Cu") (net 17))
 (segment (start 113.6725 95.59) (end 114.5125 94.75) (width 0.25) (layer "F.Cu") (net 17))
 (segment (start 112.1975 95.59) (end 113.6725 95.59) (width 0.25) (layer "F.Cu") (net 17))
 (segment (start 120.75 96.5) (end 121 96.25) (width 0.25) (layer "F.Cu") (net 9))
 (segment (start 121 96.25) (end 124.5 96.25) (width 0.25) (layer "F.Cu") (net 9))
 (segment (start 102.75 89) (end 102.34 88.59) (width 0.25) (layer "F.Cu") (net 9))
 (segment (start 102.34 88.59) (end 99.6075 88.59) (width 0.25) (layer "F.Cu") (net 9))
 (via blind (at 120.75 96.5) (size 0.8) (drill 0.4) (layers "F.Cu" "B.Cu") (free) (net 9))
 (via blind (at 102.75 89) (size 0.8) (drill 0.4) (layers "F.Cu" "B.Cu") (free) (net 9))
 (segment (start 114.025 103.225) (end 113.199695 103.225) (width 0.25) (layer "B.Cu") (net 9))
 (segment (start 102.75 92.775305) (end 102.75 89) (width 0.25) (layer "B.Cu") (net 9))
 (segment (start 120.75 96.5) (end 114.025 103.225) (width 0.25) (layer "B.Cu") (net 9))
 (segment (start 113.199695 103.225) (end 102.75 92.775305) (width 0.25) (layer "B.Cu") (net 9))
 (segment (start 131.75 114.75) (end 133 113.5) (width 0.25) (layer "F.Cu") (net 1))
 (segment (start 139.25 97.75) (end 142 97.75) (width 0.25) (layer "F.Cu") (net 1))
 (segment (start 130.25 114.75) (end 131.75 114.75) (width 0.25) (layer "F.Cu") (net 1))
 (via blind (at 133 113.5) (size 0.8) (drill 0.4) (layers "F.Cu" "B.Cu") (free) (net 1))
 (via blind (at 139.25 97.75) (size 0.8) (drill 0.4) (layers "F.Cu" "B.Cu") (free) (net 1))
 (segment (start 142.975 101.475) (end 139.25 97.75) (width 0.25) (layer "B.Cu") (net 1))
 (segment (start 133 113.5) (end 135.025 111.475) (width 0.25) (layer "B.Cu") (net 1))
 (segment (start 135.025 111.475) (end 142.550305 111.475) (width 0.25) (layer "B.Cu") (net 1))
 (segment (start 142.975 111.050305) (end 142.975 101.475) (width 0.25) (layer "B.Cu") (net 1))
 (segment (start 142.550305 111.475) (end 142.975 111.050305) (width 0.25) (layer "B.Cu") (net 1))
 (segment (start 146.55 108.38) (end 146.55 100.05) (width 0.25) (layer "F.Cu") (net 27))
 (segment (start 142.75 96.25) (end 142 96.25) (width 0.25) (layer "F.Cu") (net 27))
 (segment (start 149.75 111.58) (end 146.55 108.38) (width 0.25) (layer "F.Cu") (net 27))
 (segment (start 146.55 100.05) (end 142.75 96.25) (width 0.25) (layer "F.Cu") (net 27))
 (segment (start 149.75 109.04) (end 147 106.29) (width 0.25) (layer "F.Cu") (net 28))
 (segment (start 142.3 94.75) (end 142 94.75) (width 0.25) (layer "F.Cu") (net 28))
 (segment (start 147 99.45) (end 142.3 94.75) (width 0.25) (layer "F.Cu") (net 28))
 (segment (start 147 106.29) (end 147 99.45) (width 0.25) (layer "F.Cu") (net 28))
 (segment (start 143.87 85.75) (end 142 85.75) (width 0.25) (layer "F.Cu") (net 22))
 (segment (start 149.75 91.63) (end 143.87 85.75) (width 0.25) (layer "F.Cu") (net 22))
 (segment (start 149.75 94.17) (end 142.83 87.25) (width 0.25) (layer "F.Cu") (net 23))
 (segment (start 142.83 87.25) (end 142 87.25) (width 0.25) (layer "F.Cu") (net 23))
 (segment (start 149.75 96.15) (end 142.35 88.75) (width 0.25) (layer "F.Cu") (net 24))
 (segment (start 149.75 96.71) (end 149.75 96.15) (width 0.25) (layer "F.Cu") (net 24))
 (segment (start 142.35 88.75) (end 142 88.75) (width 0.25) (layer "F.Cu") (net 24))
 (segment (start 149.75 99.25) (end 143.075 92.575) (width 0.25) (layer "F.Cu") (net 25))
 (segment (start 142.3 90.25) (end 142 90.25) (width 0.25) (layer "F.Cu") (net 25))
 (segment (start 143.075 91.025) (end 142.3 90.25) (width 0.25) (layer "F.Cu") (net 25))
 (segment (start 143.075 92.575) (end 143.075 91.025) (width 0.25) (layer "F.Cu") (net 25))
 (segment (start 106.6025 106.1875) (end 106.6025 97.885) (width 0.25) (layer "F.Cu") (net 14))
 (segment (start 103.04 109.75) (end 106.6025 106.1875) (width 0.25) (layer "F.Cu") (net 14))
 (segment (start 102.60901 110.7905) (end 101.9995 110.18099) (width 0.25) (layer "F.Cu") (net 3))
 (segment (start 105.2025 101.2975) (end 105.2025 97.885) (width 0.25) (layer "F.Cu") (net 3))
 (segment (start 101.9995 110.18099) (end 101.9995 104.5005) (width 0.25) (layer "F.Cu") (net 3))
 (segment (start 109.4195 110.7905) (end 102.60901 110.7905) (width 0.25) (layer "F.Cu") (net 3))
 (segment (start 110.46 109.75) (end 109.4195 110.7905) (width 0.25) (layer "F.Cu") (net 3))
 (segment (start 101.9995 104.5005) (end 105.2025 101.2975) (width 0.25) (layer "F.Cu") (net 3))
 (segment (start 112.1975 88.59) (end 109.41 88.59) (width 0.25) (layer "F.Cu") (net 21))
 (segment (start 109.41 88.59) (end 109.25 88.75) (width 0.25) (layer "F.Cu") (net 21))
 (segment (start 113.5 102.5) (end 115.95 102.5) (width 0.25) (layer "F.Cu") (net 21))
 (via blind (at 109.25 88.75) (size 0.8) (drill 0.4) (layers "F.Cu" "B.Cu") (free) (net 21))
 (via blind (at 113.5 102.5) (size 0.8) (drill 0.4) (layers "F.Cu" "B.Cu") (free) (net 21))
 (segment (start 109.25 88.75) (end 109.25 98.25) (width 0.25) (layer "B.Cu") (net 21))
 (segment (start 109.25 98.25) (end 113.5 102.5) (width 0.25) (layer "B.Cu") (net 21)))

